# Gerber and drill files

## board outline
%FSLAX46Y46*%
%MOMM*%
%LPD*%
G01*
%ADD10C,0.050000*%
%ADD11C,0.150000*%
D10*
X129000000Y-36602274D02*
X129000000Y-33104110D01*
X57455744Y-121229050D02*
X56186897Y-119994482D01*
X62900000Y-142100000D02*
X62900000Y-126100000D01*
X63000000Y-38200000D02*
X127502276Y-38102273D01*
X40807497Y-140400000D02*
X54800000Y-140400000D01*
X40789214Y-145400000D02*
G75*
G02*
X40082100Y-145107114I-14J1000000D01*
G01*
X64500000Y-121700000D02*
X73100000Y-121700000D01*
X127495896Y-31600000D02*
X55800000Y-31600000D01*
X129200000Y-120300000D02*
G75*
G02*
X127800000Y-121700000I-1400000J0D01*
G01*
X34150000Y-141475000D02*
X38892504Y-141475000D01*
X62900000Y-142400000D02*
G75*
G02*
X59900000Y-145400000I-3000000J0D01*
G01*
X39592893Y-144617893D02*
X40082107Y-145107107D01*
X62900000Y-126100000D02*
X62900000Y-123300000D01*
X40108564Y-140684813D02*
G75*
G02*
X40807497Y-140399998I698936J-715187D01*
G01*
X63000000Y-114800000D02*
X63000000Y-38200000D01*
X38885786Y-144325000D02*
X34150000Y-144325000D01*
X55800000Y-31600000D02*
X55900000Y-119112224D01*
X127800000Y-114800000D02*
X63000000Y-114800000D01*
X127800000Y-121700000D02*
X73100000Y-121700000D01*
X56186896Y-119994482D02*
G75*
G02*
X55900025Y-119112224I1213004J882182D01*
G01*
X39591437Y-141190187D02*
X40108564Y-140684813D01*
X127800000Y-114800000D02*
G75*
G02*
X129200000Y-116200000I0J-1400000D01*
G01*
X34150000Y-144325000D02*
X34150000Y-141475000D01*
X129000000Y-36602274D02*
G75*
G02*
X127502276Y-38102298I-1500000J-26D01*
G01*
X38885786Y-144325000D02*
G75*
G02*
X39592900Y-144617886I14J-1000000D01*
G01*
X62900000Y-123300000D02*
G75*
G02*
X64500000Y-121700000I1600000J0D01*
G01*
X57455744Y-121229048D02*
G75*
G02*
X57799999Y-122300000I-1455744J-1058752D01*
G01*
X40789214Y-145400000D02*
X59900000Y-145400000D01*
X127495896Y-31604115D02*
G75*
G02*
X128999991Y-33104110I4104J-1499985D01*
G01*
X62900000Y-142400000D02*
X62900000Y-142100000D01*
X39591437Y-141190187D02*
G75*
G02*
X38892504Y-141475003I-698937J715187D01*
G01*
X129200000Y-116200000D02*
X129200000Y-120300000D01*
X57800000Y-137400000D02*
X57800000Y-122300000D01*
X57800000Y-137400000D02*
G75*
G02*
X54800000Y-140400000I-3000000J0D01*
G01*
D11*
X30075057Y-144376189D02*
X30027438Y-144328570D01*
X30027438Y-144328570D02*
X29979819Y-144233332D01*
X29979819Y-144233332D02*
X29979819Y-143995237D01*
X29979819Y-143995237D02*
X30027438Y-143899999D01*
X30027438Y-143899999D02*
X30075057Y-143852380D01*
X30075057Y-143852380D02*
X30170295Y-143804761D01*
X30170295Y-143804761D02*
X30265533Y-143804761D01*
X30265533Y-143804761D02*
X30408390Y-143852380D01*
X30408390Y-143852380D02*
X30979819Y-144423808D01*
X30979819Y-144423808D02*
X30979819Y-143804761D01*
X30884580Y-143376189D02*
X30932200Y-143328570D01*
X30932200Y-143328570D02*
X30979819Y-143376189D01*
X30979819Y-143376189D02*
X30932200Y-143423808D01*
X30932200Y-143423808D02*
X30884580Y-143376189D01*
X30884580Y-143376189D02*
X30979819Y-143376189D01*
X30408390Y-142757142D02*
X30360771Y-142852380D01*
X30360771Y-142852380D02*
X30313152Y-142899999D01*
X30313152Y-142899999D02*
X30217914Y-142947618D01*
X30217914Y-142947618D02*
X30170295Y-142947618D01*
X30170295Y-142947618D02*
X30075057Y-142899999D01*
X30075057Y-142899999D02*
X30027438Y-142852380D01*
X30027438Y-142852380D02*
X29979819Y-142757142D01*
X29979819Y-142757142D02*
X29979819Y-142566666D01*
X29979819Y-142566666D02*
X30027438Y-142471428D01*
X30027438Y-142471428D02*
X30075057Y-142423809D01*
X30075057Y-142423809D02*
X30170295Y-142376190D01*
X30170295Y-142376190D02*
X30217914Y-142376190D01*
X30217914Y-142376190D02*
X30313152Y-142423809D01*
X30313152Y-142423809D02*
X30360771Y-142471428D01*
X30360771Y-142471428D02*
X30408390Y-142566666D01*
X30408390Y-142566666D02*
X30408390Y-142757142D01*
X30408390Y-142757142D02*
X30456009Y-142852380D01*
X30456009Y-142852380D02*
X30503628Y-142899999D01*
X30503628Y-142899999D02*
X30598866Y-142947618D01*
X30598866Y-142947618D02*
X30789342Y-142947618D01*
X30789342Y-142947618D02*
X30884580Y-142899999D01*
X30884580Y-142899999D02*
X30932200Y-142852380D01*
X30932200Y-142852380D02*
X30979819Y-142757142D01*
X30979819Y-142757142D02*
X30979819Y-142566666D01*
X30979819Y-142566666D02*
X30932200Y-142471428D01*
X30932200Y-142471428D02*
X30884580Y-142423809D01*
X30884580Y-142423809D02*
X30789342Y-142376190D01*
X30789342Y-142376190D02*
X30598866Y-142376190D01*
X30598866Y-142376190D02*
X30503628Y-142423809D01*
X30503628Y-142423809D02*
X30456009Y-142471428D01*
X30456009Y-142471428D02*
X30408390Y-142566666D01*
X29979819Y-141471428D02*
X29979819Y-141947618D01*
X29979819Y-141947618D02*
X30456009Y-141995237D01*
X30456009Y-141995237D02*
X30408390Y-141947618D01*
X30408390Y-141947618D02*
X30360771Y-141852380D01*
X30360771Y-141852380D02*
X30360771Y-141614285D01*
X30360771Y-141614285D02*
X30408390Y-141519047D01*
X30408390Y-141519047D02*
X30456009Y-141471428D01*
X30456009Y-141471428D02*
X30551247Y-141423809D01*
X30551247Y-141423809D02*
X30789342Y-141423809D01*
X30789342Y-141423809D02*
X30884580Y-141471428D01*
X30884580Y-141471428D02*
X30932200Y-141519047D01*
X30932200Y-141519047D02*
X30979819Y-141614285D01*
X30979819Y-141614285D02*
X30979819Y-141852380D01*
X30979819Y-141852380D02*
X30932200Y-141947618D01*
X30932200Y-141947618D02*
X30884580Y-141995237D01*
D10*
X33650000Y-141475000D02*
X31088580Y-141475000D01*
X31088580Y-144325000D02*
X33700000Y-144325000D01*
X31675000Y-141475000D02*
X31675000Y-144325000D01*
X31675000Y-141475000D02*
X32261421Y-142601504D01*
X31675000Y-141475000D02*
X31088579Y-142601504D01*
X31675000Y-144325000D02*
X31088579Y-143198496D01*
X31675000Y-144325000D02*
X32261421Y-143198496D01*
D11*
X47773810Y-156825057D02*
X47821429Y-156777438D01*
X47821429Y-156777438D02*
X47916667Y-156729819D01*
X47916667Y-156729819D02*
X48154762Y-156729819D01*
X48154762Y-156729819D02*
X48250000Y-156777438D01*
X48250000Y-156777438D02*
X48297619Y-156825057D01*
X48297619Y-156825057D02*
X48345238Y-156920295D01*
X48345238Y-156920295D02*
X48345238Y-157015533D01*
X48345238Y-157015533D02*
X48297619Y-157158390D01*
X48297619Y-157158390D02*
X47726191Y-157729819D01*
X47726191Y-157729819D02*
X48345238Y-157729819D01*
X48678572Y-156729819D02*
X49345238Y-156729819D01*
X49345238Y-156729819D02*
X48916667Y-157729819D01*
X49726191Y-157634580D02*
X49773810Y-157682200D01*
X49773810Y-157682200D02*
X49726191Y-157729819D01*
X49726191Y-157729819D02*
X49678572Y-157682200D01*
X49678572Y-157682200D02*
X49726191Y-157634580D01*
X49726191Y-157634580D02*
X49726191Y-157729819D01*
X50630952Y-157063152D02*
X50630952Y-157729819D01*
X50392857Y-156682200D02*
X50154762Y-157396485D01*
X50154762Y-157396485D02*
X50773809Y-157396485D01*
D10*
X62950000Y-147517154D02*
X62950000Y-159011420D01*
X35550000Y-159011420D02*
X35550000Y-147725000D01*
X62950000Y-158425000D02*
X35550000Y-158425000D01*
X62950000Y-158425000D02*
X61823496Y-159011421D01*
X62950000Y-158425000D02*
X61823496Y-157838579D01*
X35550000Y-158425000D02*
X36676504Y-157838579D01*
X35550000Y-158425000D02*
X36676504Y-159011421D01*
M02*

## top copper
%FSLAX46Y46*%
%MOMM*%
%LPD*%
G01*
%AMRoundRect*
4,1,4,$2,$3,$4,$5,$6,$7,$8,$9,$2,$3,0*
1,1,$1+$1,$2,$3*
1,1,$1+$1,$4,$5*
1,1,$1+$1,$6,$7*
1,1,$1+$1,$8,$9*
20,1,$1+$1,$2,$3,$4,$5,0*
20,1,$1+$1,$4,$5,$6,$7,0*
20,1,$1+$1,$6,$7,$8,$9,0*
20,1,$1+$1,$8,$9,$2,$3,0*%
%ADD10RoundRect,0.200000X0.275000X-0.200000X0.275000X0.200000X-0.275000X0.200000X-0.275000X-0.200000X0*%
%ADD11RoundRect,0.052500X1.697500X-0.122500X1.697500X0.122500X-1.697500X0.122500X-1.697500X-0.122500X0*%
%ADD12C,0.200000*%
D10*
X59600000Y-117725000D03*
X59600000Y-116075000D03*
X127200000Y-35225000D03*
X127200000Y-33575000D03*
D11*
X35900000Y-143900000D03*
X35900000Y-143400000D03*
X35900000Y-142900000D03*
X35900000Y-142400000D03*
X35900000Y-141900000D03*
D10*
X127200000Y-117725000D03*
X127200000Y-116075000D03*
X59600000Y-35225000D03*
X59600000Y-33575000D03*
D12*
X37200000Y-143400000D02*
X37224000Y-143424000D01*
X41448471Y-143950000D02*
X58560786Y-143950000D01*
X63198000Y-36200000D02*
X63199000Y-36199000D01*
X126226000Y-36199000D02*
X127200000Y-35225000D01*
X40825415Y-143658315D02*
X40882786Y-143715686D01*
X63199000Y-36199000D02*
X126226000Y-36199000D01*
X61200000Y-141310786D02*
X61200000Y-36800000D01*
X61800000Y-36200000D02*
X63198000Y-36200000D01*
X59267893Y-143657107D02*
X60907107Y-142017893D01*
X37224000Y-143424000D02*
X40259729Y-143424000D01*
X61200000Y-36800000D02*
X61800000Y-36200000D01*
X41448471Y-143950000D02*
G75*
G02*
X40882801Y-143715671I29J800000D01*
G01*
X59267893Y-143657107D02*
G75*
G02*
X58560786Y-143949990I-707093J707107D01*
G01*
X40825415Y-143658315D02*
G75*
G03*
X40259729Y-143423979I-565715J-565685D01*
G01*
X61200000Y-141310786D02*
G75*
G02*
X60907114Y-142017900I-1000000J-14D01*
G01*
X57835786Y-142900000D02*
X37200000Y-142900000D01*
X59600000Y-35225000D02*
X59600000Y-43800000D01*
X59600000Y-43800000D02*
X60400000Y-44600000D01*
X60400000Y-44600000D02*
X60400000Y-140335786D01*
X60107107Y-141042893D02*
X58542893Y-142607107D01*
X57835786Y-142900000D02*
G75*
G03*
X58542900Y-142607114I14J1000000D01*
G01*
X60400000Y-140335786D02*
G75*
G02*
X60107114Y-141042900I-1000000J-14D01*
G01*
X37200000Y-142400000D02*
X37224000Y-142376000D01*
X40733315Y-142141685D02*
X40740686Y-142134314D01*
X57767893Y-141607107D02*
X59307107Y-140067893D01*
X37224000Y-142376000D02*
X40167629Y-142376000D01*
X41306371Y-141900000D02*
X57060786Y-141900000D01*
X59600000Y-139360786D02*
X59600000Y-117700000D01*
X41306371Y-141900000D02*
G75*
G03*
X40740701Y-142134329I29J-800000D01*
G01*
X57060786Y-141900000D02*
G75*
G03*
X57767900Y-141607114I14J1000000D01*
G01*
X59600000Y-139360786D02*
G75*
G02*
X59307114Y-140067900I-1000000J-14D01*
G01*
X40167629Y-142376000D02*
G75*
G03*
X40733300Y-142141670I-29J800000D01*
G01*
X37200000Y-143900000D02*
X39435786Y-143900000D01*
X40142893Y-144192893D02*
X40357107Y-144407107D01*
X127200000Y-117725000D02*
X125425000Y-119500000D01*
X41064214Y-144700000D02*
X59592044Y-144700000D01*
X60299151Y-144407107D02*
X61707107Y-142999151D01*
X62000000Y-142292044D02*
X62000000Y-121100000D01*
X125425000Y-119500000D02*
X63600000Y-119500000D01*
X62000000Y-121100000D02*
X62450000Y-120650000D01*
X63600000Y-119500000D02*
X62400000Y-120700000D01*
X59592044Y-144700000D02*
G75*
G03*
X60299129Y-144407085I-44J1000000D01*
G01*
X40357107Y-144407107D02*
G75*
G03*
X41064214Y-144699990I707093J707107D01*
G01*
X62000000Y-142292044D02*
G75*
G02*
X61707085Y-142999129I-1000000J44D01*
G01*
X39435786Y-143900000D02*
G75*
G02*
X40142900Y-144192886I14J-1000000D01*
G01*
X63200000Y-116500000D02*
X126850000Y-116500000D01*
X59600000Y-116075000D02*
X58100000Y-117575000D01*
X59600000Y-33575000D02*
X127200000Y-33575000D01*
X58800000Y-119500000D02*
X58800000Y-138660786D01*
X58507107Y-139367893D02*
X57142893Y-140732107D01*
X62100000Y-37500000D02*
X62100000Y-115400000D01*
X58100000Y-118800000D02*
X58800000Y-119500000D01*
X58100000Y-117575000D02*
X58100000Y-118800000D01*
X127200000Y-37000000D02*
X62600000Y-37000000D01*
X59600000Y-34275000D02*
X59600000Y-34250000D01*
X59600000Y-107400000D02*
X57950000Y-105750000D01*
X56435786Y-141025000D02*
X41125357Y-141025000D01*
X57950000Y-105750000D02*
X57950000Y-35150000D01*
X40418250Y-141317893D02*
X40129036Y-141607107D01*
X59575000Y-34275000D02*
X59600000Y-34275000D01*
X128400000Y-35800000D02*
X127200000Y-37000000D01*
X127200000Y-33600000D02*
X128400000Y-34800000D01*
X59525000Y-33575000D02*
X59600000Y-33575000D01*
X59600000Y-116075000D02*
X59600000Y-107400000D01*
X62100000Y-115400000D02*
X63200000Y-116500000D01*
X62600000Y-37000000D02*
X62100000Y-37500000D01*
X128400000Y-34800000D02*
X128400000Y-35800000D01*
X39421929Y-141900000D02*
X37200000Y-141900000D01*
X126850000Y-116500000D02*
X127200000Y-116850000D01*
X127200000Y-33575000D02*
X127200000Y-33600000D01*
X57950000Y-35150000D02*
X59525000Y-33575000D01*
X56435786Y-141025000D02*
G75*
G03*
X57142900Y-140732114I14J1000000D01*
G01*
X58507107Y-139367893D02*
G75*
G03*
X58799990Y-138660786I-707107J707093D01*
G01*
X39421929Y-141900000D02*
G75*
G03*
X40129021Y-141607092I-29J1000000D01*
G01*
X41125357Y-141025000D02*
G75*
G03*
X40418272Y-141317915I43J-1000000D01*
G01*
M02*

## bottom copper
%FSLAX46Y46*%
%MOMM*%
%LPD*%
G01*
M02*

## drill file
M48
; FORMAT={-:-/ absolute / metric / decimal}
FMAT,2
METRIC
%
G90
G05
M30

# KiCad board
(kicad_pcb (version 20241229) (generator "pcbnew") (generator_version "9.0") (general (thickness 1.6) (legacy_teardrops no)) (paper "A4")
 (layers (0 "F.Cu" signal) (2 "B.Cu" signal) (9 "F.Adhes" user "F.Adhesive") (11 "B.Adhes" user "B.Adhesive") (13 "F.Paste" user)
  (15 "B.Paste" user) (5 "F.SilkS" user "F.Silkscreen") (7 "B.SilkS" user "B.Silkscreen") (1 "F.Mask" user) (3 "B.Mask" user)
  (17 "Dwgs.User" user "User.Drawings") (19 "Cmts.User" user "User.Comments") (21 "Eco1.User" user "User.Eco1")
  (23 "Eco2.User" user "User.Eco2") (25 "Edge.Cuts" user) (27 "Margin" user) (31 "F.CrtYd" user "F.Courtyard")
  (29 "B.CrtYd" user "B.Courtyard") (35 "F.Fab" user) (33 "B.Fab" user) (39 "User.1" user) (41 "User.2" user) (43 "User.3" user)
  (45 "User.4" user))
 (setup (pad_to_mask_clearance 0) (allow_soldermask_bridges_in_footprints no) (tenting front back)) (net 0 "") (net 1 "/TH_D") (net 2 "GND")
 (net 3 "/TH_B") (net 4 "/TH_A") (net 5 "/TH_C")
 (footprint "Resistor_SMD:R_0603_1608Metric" (layer "F.Cu") (at 59.6 116.9 90)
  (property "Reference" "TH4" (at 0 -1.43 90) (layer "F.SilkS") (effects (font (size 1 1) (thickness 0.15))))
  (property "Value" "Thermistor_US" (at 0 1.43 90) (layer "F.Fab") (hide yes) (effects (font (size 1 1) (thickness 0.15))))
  (pad "1" smd roundrect (at -0.825 0 90) (size 0.8 0.95) (layers "F.Cu" "F.Mask" "F.Paste") (roundrect_rratio 0.25) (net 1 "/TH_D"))
  (pad "2" smd roundrect (at 0.825 0 90) (size 0.8 0.95) (layers "F.Cu" "F.Mask" "F.Paste") (roundrect_rratio 0.25) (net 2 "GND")))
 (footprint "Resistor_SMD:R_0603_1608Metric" (layer "F.Cu") (at 127.2 34.4 90)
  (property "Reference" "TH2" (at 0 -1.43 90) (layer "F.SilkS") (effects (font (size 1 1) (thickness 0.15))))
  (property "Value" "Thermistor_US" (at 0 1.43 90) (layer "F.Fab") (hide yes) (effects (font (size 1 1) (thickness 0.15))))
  (pad "1" smd roundrect (at -0.825 0 90) (size 0.8 0.95) (layers "F.Cu" "F.Mask" "F.Paste") (roundrect_rratio 0.25) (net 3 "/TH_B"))
  (pad "2" smd roundrect (at 0.825 0 90) (size 0.8 0.95) (layers "F.Cu" "F.Mask" "F.Paste") (roundrect_rratio 0.25) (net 2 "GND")))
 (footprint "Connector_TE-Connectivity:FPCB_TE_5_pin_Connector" (layer "F.Cu") (at 34.15 142.9 90)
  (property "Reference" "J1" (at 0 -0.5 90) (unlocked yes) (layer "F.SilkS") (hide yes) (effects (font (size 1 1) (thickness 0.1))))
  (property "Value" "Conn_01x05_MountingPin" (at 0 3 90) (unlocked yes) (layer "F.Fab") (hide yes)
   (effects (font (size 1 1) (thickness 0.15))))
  (pad "1" smd roundrect (at -1 1.75 90) (size 0.35 3.5) (layers "F.Cu" "F.Mask" "F.Paste") (roundrect_rratio 0.15) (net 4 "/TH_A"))
  (pad "2" smd roundrect (at -0.5 1.75 90) (size 0.35 3.5) (layers "F.Cu" "F.Mask" "F.Paste") (roundrect_rratio 0.15) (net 3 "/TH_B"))
  (pad "3" smd roundrect (at 0 1.75 90) (size 0.35 3.5) (layers "F.Cu" "F.Mask" "F.Paste") (roundrect_rratio 0.15) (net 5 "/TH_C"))
  (pad "4" smd roundrect (at 0.5 1.75 90) (size 0.35 3.5) (layers "F.Cu" "F.Mask" "F.Paste") (roundrect_rratio 0.15) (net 1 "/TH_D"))
  (pad "5" smd roundrect (at 1 1.75 90) (size 0.35 3.5) (layers "F.Cu" "F.Mask" "F.Paste") (roundrect_rratio 0.15) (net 2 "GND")))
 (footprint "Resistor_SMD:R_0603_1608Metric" (layer "F.Cu") (at 127.2 116.9 90)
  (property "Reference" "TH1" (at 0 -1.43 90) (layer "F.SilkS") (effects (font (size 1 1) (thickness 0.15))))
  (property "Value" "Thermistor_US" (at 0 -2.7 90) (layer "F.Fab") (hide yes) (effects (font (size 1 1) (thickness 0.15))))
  (pad "1" smd roundrect (at -0.825 0 90) (size 0.8 0.95) (layers "F.Cu" "F.Mask" "F.Paste") (roundrect_rratio 0.25) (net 4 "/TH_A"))
  (pad "2" smd roundrect (at 0.825 0 90) (size 0.8 0.95) (layers "F.Cu" "F.Mask" "F.Paste") (roundrect_rratio 0.25) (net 2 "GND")))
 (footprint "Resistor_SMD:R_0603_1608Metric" (layer "F.Cu") (at 59.6 34.4 90)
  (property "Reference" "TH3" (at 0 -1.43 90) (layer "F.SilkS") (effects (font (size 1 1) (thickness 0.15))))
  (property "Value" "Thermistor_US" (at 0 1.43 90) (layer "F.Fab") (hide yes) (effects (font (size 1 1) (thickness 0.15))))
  (pad "1" smd roundrect (at -0.825 0 90) (size 0.8 0.95) (layers "F.Cu" "F.Mask" "F.Paste") (roundrect_rratio 0.25) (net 5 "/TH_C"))
  (pad "2" smd roundrect (at 0.825 0 90) (size 0.8 0.95) (layers "F.Cu" "F.Mask" "F.Paste") (roundrect_rratio 0.25) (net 2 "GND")))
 (gr_line (start 129 36.602274) (end 129 33.10411) (stroke (width 0.05) (type default)) (layer "Edge.Cuts"))
 (gr_line (start 57.455744 121.22905) (end 56.186897 119.994482) (stroke (width 0.05) (type default)) (layer "Edge.Cuts"))
 (gr_line (start 62.9 142.1) (end 62.9 126.1) (stroke (width 0.05) (type default)) (layer "Edge.Cuts"))
 (gr_line (start 63 38.2) (end 127.502276 38.102273) (stroke (width 0.05) (type default)) (layer "Edge.Cuts"))
 (gr_line (start 40.807497 140.4) (end 54.8 140.4) (stroke (width 0.05) (type default)) (layer "Edge.Cuts"))
 (gr_arc (start 40.789214 145.4) (mid 40.406531 145.32388) (end 40.082107 145.107107) (stroke (width 0.05) (type default))
  (layer "Edge.Cuts"))
 (gr_line (start 64.5 121.7) (end 73.1 121.7) (stroke (width 0.05) (type default)) (layer "Edge.Cuts"))
 (gr_line (start 127.495896 31.6) (end 55.8 31.6) (stroke (width 0.05) (type solid)) (layer "Edge.Cuts"))
 (gr_arc (start 129.2 120.3) (mid 128.789949 121.289949) (end 127.8 121.7) (stroke (width 0.05) (type default)) (layer "Edge.Cuts"))
 (gr_line (start 34.15 141.475) (end 38.892504 141.475) (stroke (width 0.05) (type default)) (layer "Edge.Cuts"))
 (gr_arc (start 62.9 142.4) (mid 62.02132 144.52132) (end 59.9 145.4) (stroke (width 0.05) (type default)) (layer "Edge.Cuts"))
 (gr_line (start 39.592893 144.617893) (end 40.082107 145.107107) (stroke (width 0.05) (type default)) (layer "Edge.Cuts"))
 (gr_line (start 62.9 126.1) (end 62.9 123.3) (stroke (width 0.05) (type default)) (layer "Edge.Cuts"))
 (gr_arc (start 40.108564 140.684813) (mid 40.430129 140.473936) (end 40.807497 140.4) (stroke (width 0.05) (type default))
  (layer "Edge.Cuts"))
 (gr_line (start 63 114.8) (end 63 38.2) (stroke (width 0.05) (type solid)) (layer "Edge.Cuts"))
 (gr_line (start 38.885786 144.325) (end 34.15 144.325) (stroke (width 0.05) (type solid)) (layer "Edge.Cuts"))
 (gr_line (start 55.8 31.6) (end 55.9 119.112224) (stroke (width 0.05) (type default)) (layer "Edge.Cuts"))
 (gr_line (start 127.8 114.8) (end 63 114.8) (stroke (width 0.05) (type default)) (layer "Edge.Cuts"))
 (gr_line (start 127.8 121.7) (end 73.1 121.7) (stroke (width 0.05) (type default)) (layer "Edge.Cuts"))
 (gr_arc (start 56.186896 119.994482) (mid 55.973519 119.576092) (end 55.9 119.112224) (stroke (width 0.05) (type default))
  (layer "Edge.Cuts"))
 (gr_line (start 39.591437 141.190187) (end 40.108564 140.684813) (stroke (width 0.05) (type default)) (layer "Edge.Cuts"))
 (gr_arc (start 127.8 114.8) (mid 128.789949 115.210051) (end 129.2 116.2) (stroke (width 0.05) (type default)) (layer "Edge.Cuts"))
 (gr_line (start 34.15 144.325) (end 34.15 141.475) (stroke (width 0.05) (type default)) (layer "Edge.Cuts"))
 (gr_arc (start 129 36.602274) (mid 128.561474 37.662146) (end 127.502276 38.102273) (stroke (width 0.05) (type default))
  (layer "Edge.Cuts"))
 (gr_arc (start 38.885786 144.325) (mid 39.268469 144.40112) (end 39.592893 144.617893) (stroke (width 0.05) (type default))
  (layer "Edge.Cuts"))
 (gr_arc (start 62.9 123.3) (mid 63.368629 122.168629) (end 64.5 121.7) (stroke (width 0.05) (type default)) (layer "Edge.Cuts"))
 (gr_arc (start 57.455744 121.229048) (mid 57.71368 121.736941) (end 57.8 122.3) (stroke (width 0.05) (type default)) (layer "Edge.Cuts"))
 (gr_line (start 40.789214 145.4) (end 59.9 145.4) (stroke (width 0.05) (type default)) (layer "Edge.Cuts"))
 (gr_arc (start 127.495896 31.604115) (mid 128.559209 32.041999) (end 129 33.10411) (stroke (width 0.05) (type default)) (layer "Edge.Cuts"))
 (gr_line (start 62.9 142.4) (end 62.9 142.1) (stroke (width 0.05) (type default)) (layer "Edge.Cuts"))
 (gr_arc (start 39.591437 141.190187) (mid 39.269872 141.401063) (end 38.892504 141.475) (stroke (width 0.05) (type default))
  (layer "Edge.Cuts"))
 (gr_line (start 129.2 116.2) (end 129.2 120.3) (stroke (width 0.05) (type default)) (layer "Edge.Cuts"))
 (gr_line (start 57.8 137.4) (end 57.8 122.3) (stroke (width 0.05) (type solid)) (layer "Edge.Cuts"))
 (gr_arc (start 57.8 137.4) (mid 56.92132 139.52132) (end 54.8 140.4) (stroke (width 0.05) (type default)) (layer "Edge.Cuts"))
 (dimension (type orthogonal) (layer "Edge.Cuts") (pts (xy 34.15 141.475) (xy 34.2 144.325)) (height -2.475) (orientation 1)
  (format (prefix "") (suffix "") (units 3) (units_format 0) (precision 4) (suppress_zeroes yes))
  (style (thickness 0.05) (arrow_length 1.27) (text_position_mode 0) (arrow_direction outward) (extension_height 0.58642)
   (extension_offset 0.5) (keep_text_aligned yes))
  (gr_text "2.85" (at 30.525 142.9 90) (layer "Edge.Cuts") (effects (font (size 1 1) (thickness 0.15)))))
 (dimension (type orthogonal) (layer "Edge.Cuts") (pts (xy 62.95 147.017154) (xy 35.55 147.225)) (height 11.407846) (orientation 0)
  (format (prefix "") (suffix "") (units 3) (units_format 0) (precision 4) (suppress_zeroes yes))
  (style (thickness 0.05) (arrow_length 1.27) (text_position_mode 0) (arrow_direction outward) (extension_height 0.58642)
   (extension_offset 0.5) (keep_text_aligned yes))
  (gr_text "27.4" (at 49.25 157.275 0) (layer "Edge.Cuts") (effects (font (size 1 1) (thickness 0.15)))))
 (segment (start 37.2 143.4) (end 37.224 143.424) (width 0.2) (layer "F.Cu") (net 3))
 (segment (start 41.448471 143.95) (end 58.560786 143.95) (width 0.2) (layer "F.Cu") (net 3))
 (segment (start 63.198 36.2) (end 63.199 36.199) (width 0.2) (layer "F.Cu") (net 3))
 (segment (start 126.226 36.199) (end 127.2 35.225) (width 0.2) (layer "F.Cu") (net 3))
 (segment (start 40.825415 143.658315) (end 40.882786 143.715686) (width 0.2) (layer "F.Cu") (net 3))
 (segment (start 63.199 36.199) (end 126.226 36.199) (width 0.2) (layer "F.Cu") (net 3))
 (segment (start 61.2 141.310786) (end 61.2 36.8) (width 0.2) (layer "F.Cu") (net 3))
 (segment (start 61.8 36.2) (end 63.198 36.2) (width 0.2) (layer "F.Cu") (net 3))
 (segment (start 59.267893 143.657107) (end 60.907107 142.017893) (width 0.2) (layer "F.Cu") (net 3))
 (segment (start 37.224 143.424) (end 40.259729 143.424) (width 0.2) (layer "F.Cu") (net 3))
 (segment (start 61.2 36.8) (end 61.8 36.2) (width 0.2) (layer "F.Cu") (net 3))
 (arc (start 41.448471 143.95) (mid 41.142325 143.889104) (end 40.882786 143.715686) (width 0.2) (layer "F.Cu") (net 3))
 (arc (start 59.267893 143.657107) (mid 58.94347 143.87388) (end 58.560786 143.95) (width 0.2) (layer "F.Cu") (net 3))
 (arc (start 40.825415 143.658315) (mid 40.565876 143.484896) (end 40.259729 143.424) (width 0.2) (layer "F.Cu") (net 3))
 (arc (start 61.2 141.310786) (mid 61.12388 141.693469) (end 60.907107 142.017893) (width 0.2) (layer "F.Cu") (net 3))
 (segment (start 57.835786 142.9) (end 37.2 142.9) (width 0.2) (layer "F.Cu") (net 5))
 (segment (start 59.6 35.225) (end 59.6 43.8) (width 0.2) (layer "F.Cu") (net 5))
 (segment (start 59.6 43.8) (end 60.4 44.6) (width 0.2) (layer "F.Cu") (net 5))
 (segment (start 60.4 44.6) (end 60.4 140.335786) (width 0.2) (layer "F.Cu") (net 5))
 (segment (start 60.107107 141.042893) (end 58.542893 142.607107) (width 0.2) (layer "F.Cu") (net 5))
 (arc (start 57.835786 142.9) (mid 58.218469 142.82388) (end 58.542893 142.607107) (width 0.2) (layer "F.Cu") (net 5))
 (arc (start 60.4 140.335786) (mid 60.32388 140.718469) (end 60.107107 141.042893) (width 0.2) (layer "F.Cu") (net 5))
 (segment (start 37.2 142.4) (end 37.224 142.376) (width 0.2) (layer "F.Cu") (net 1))
 (segment (start 40.733315 142.141685) (end 40.740686 142.134314) (width 0.2) (layer "F.Cu") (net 1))
 (segment (start 57.767893 141.607107) (end 59.307107 140.067893) (width 0.2) (layer "F.Cu") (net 1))
 (segment (start 37.224 142.376) (end 40.167629 142.376) (width 0.2) (layer "F.Cu") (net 1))
 (segment (start 41.306371 141.9) (end 57.060786 141.9) (width 0.2) (layer "F.Cu") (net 1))
 (segment (start 59.6 139.360786) (end 59.6 117.7) (width 0.2) (layer "F.Cu") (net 1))
 (arc (start 41.306371 141.9) (mid 41.000225 141.960896) (end 40.740686 142.134314) (width 0.2) (layer "F.Cu") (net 1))
 (arc (start 57.060786 141.9) (mid 57.443469 141.82388) (end 57.767893 141.607107) (width 0.2) (layer "F.Cu") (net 1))
 (arc (start 59.6 139.360786) (mid 59.52388 139.743469) (end 59.307107 140.067893) (width 0.2) (layer "F.Cu") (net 1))
 (arc (start 40.167629 142.376) (mid 40.473776 142.315103) (end 40.733315 142.141685) (width 0.2) (layer "F.Cu") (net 1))
 (segment (start 37.2 143.9) (end 39.435786 143.9) (width 0.2) (layer "F.Cu") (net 4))
 (segment (start 40.142893 144.192893) (end 40.357107 144.407107) (width 0.2) (layer "F.Cu") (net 4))
 (segment (start 127.2 117.725) (end 125.425 119.5) (width 0.2) (layer "F.Cu") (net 4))
 (segment (start 41.064214 144.7) (end 59.592044 144.7) (width 0.2) (layer "F.Cu") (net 4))
 (segment (start 60.299151 144.407107) (end 61.707107 142.999151) (width 0.2) (layer "F.Cu") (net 4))
 (segment (start 62 142.292044) (end 62 121.1) (width 0.2) (layer "F.Cu") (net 4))
 (segment (start 125.425 119.5) (end 63.6 119.5) (width 0.2) (layer "F.Cu") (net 4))
 (segment (start 62 121.1) (end 62.45 120.65) (width 0.2) (layer "F.Cu") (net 4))
 (segment (start 63.6 119.5) (end 62.4 120.7) (width 0.2) (layer "F.Cu") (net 4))
 (arc (start 59.592044 144.7) (mid 59.974727 144.62388) (end 60.299151 144.407107) (width 0.2) (layer "F.Cu") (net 4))
 (arc (start 40.357107 144.407107) (mid 40.681531 144.62388) (end 41.064214 144.7) (width 0.2) (layer "F.Cu") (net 4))
 (arc (start 62 142.292044) (mid 61.92388 142.674727) (end 61.707107 142.999151) (width 0.2) (layer "F.Cu") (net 4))
 (arc (start 39.435786 143.9) (mid 39.818469 143.97612) (end 40.142893 144.192893) (width 0.2) (layer "F.Cu") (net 4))
 (segment (start 63.2 116.5) (end 126.85 116.5) (width 0.2) (layer "F.Cu") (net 2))
 (segment (start 59.6 116.075) (end 58.1 117.575) (width 0.2) (layer "F.Cu") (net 2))
 (segment (start 59.6 33.575) (end 127.2 33.575) (width 0.2) (layer "F.Cu") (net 2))
 (segment (start 58.8 119.5) (end 58.8 138.660786) (width 0.2) (layer "F.Cu") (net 2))
 (segment (start 58.507107 139.367893) (end 57.142893 140.732107) (width 0.2) (layer "F.Cu") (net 2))
 (segment (start 62.1 37.5) (end 62.1 115.4) (width 0.2) (layer "F.Cu") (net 2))
 (segment (start 58.1 118.8) (end 58.8 119.5) (width 0.2) (layer "F.Cu") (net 2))
 (segment (start 58.1 117.575) (end 58.1 118.8) (width 0.2) (layer "F.Cu") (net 2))
 (segment (start 127.2 37) (end 62.6 37) (width 0.2) (layer "F.Cu") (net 2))
 (segment (start 59.6 34.275) (end 59.6 34.25) (width 0.2) (layer "F.Cu") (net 2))
 (segment (start 59.6 107.4) (end 57.95 105.75) (width 0.2) (layer "F.Cu") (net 2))
 (segment (start 56.435786 141.025) (end 41.125357 141.025) (width 0.2) (layer "F.Cu") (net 2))
 (segment (start 57.95 105.75) (end 57.95 35.15) (width 0.2) (layer "F.Cu") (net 2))
 (segment (start 40.41825 141.317893) (end 40.129036 141.607107) (width 0.2) (layer "F.Cu") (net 2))
 (segment (start 59.575 34.275) (end 59.6 34.275) (width 0.2) (layer "F.Cu") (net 2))
 (segment (start 128.4 35.8) (end 127.2 37) (width 0.2) (layer "F.Cu") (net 2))
 (segment (start 127.2 33.6) (end 128.4 34.8) (width 0.2) (layer "F.Cu") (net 2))
 (segment (start 59.525 33.575) (end 59.6 33.575) (width 0.2) (layer "F.Cu") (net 2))
 (segment (start 59.6 116.075) (end 59.6 107.4) (width 0.2) (layer "F.Cu") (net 2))
 (segment (start 62.1 115.4) (end 63.2 116.5) (width 0.2) (layer "F.Cu") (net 2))
 (segment (start 62.6 37) (end 62.1 37.5) (width 0.2) (layer "F.Cu") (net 2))
 (segment (start 128.4 34.8) (end 128.4 35.8) (width 0.2) (layer "F.Cu") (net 2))
 (segment (start 39.421929 141.9) (end 37.2 141.9) (width 0.2) (layer "F.Cu") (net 2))
 (segment (start 126.85 116.5) (end 127.2 116.85) (width 0.2) (layer "F.Cu") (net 2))
 (segment (start 127.2 33.575) (end 127.2 33.6) (width 0.2) (layer "F.Cu") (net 2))
 (segment (start 57.95 35.15) (end 59.525 33.575) (width 0.2) (layer "F.Cu") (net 2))
 (arc (start 56.435786 141.025) (mid 56.818469 140.94888) (end 57.142893 140.732107) (width 0.2) (layer "F.Cu") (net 2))
 (arc (start 58.507107 139.367893) (mid 58.72388 139.04347) (end 58.8 138.660786) (width 0.2) (layer "F.Cu") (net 2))
 (arc (start 39.421929 141.9) (mid 39.804612 141.82388) (end 40.129036 141.607107) (width 0.2) (layer "F.Cu") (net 2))
 (arc (start 41.125357 141.025) (mid 40.742674 141.10112) (end 40.41825 141.317893) (width 0.2) (layer "F.Cu") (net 2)))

